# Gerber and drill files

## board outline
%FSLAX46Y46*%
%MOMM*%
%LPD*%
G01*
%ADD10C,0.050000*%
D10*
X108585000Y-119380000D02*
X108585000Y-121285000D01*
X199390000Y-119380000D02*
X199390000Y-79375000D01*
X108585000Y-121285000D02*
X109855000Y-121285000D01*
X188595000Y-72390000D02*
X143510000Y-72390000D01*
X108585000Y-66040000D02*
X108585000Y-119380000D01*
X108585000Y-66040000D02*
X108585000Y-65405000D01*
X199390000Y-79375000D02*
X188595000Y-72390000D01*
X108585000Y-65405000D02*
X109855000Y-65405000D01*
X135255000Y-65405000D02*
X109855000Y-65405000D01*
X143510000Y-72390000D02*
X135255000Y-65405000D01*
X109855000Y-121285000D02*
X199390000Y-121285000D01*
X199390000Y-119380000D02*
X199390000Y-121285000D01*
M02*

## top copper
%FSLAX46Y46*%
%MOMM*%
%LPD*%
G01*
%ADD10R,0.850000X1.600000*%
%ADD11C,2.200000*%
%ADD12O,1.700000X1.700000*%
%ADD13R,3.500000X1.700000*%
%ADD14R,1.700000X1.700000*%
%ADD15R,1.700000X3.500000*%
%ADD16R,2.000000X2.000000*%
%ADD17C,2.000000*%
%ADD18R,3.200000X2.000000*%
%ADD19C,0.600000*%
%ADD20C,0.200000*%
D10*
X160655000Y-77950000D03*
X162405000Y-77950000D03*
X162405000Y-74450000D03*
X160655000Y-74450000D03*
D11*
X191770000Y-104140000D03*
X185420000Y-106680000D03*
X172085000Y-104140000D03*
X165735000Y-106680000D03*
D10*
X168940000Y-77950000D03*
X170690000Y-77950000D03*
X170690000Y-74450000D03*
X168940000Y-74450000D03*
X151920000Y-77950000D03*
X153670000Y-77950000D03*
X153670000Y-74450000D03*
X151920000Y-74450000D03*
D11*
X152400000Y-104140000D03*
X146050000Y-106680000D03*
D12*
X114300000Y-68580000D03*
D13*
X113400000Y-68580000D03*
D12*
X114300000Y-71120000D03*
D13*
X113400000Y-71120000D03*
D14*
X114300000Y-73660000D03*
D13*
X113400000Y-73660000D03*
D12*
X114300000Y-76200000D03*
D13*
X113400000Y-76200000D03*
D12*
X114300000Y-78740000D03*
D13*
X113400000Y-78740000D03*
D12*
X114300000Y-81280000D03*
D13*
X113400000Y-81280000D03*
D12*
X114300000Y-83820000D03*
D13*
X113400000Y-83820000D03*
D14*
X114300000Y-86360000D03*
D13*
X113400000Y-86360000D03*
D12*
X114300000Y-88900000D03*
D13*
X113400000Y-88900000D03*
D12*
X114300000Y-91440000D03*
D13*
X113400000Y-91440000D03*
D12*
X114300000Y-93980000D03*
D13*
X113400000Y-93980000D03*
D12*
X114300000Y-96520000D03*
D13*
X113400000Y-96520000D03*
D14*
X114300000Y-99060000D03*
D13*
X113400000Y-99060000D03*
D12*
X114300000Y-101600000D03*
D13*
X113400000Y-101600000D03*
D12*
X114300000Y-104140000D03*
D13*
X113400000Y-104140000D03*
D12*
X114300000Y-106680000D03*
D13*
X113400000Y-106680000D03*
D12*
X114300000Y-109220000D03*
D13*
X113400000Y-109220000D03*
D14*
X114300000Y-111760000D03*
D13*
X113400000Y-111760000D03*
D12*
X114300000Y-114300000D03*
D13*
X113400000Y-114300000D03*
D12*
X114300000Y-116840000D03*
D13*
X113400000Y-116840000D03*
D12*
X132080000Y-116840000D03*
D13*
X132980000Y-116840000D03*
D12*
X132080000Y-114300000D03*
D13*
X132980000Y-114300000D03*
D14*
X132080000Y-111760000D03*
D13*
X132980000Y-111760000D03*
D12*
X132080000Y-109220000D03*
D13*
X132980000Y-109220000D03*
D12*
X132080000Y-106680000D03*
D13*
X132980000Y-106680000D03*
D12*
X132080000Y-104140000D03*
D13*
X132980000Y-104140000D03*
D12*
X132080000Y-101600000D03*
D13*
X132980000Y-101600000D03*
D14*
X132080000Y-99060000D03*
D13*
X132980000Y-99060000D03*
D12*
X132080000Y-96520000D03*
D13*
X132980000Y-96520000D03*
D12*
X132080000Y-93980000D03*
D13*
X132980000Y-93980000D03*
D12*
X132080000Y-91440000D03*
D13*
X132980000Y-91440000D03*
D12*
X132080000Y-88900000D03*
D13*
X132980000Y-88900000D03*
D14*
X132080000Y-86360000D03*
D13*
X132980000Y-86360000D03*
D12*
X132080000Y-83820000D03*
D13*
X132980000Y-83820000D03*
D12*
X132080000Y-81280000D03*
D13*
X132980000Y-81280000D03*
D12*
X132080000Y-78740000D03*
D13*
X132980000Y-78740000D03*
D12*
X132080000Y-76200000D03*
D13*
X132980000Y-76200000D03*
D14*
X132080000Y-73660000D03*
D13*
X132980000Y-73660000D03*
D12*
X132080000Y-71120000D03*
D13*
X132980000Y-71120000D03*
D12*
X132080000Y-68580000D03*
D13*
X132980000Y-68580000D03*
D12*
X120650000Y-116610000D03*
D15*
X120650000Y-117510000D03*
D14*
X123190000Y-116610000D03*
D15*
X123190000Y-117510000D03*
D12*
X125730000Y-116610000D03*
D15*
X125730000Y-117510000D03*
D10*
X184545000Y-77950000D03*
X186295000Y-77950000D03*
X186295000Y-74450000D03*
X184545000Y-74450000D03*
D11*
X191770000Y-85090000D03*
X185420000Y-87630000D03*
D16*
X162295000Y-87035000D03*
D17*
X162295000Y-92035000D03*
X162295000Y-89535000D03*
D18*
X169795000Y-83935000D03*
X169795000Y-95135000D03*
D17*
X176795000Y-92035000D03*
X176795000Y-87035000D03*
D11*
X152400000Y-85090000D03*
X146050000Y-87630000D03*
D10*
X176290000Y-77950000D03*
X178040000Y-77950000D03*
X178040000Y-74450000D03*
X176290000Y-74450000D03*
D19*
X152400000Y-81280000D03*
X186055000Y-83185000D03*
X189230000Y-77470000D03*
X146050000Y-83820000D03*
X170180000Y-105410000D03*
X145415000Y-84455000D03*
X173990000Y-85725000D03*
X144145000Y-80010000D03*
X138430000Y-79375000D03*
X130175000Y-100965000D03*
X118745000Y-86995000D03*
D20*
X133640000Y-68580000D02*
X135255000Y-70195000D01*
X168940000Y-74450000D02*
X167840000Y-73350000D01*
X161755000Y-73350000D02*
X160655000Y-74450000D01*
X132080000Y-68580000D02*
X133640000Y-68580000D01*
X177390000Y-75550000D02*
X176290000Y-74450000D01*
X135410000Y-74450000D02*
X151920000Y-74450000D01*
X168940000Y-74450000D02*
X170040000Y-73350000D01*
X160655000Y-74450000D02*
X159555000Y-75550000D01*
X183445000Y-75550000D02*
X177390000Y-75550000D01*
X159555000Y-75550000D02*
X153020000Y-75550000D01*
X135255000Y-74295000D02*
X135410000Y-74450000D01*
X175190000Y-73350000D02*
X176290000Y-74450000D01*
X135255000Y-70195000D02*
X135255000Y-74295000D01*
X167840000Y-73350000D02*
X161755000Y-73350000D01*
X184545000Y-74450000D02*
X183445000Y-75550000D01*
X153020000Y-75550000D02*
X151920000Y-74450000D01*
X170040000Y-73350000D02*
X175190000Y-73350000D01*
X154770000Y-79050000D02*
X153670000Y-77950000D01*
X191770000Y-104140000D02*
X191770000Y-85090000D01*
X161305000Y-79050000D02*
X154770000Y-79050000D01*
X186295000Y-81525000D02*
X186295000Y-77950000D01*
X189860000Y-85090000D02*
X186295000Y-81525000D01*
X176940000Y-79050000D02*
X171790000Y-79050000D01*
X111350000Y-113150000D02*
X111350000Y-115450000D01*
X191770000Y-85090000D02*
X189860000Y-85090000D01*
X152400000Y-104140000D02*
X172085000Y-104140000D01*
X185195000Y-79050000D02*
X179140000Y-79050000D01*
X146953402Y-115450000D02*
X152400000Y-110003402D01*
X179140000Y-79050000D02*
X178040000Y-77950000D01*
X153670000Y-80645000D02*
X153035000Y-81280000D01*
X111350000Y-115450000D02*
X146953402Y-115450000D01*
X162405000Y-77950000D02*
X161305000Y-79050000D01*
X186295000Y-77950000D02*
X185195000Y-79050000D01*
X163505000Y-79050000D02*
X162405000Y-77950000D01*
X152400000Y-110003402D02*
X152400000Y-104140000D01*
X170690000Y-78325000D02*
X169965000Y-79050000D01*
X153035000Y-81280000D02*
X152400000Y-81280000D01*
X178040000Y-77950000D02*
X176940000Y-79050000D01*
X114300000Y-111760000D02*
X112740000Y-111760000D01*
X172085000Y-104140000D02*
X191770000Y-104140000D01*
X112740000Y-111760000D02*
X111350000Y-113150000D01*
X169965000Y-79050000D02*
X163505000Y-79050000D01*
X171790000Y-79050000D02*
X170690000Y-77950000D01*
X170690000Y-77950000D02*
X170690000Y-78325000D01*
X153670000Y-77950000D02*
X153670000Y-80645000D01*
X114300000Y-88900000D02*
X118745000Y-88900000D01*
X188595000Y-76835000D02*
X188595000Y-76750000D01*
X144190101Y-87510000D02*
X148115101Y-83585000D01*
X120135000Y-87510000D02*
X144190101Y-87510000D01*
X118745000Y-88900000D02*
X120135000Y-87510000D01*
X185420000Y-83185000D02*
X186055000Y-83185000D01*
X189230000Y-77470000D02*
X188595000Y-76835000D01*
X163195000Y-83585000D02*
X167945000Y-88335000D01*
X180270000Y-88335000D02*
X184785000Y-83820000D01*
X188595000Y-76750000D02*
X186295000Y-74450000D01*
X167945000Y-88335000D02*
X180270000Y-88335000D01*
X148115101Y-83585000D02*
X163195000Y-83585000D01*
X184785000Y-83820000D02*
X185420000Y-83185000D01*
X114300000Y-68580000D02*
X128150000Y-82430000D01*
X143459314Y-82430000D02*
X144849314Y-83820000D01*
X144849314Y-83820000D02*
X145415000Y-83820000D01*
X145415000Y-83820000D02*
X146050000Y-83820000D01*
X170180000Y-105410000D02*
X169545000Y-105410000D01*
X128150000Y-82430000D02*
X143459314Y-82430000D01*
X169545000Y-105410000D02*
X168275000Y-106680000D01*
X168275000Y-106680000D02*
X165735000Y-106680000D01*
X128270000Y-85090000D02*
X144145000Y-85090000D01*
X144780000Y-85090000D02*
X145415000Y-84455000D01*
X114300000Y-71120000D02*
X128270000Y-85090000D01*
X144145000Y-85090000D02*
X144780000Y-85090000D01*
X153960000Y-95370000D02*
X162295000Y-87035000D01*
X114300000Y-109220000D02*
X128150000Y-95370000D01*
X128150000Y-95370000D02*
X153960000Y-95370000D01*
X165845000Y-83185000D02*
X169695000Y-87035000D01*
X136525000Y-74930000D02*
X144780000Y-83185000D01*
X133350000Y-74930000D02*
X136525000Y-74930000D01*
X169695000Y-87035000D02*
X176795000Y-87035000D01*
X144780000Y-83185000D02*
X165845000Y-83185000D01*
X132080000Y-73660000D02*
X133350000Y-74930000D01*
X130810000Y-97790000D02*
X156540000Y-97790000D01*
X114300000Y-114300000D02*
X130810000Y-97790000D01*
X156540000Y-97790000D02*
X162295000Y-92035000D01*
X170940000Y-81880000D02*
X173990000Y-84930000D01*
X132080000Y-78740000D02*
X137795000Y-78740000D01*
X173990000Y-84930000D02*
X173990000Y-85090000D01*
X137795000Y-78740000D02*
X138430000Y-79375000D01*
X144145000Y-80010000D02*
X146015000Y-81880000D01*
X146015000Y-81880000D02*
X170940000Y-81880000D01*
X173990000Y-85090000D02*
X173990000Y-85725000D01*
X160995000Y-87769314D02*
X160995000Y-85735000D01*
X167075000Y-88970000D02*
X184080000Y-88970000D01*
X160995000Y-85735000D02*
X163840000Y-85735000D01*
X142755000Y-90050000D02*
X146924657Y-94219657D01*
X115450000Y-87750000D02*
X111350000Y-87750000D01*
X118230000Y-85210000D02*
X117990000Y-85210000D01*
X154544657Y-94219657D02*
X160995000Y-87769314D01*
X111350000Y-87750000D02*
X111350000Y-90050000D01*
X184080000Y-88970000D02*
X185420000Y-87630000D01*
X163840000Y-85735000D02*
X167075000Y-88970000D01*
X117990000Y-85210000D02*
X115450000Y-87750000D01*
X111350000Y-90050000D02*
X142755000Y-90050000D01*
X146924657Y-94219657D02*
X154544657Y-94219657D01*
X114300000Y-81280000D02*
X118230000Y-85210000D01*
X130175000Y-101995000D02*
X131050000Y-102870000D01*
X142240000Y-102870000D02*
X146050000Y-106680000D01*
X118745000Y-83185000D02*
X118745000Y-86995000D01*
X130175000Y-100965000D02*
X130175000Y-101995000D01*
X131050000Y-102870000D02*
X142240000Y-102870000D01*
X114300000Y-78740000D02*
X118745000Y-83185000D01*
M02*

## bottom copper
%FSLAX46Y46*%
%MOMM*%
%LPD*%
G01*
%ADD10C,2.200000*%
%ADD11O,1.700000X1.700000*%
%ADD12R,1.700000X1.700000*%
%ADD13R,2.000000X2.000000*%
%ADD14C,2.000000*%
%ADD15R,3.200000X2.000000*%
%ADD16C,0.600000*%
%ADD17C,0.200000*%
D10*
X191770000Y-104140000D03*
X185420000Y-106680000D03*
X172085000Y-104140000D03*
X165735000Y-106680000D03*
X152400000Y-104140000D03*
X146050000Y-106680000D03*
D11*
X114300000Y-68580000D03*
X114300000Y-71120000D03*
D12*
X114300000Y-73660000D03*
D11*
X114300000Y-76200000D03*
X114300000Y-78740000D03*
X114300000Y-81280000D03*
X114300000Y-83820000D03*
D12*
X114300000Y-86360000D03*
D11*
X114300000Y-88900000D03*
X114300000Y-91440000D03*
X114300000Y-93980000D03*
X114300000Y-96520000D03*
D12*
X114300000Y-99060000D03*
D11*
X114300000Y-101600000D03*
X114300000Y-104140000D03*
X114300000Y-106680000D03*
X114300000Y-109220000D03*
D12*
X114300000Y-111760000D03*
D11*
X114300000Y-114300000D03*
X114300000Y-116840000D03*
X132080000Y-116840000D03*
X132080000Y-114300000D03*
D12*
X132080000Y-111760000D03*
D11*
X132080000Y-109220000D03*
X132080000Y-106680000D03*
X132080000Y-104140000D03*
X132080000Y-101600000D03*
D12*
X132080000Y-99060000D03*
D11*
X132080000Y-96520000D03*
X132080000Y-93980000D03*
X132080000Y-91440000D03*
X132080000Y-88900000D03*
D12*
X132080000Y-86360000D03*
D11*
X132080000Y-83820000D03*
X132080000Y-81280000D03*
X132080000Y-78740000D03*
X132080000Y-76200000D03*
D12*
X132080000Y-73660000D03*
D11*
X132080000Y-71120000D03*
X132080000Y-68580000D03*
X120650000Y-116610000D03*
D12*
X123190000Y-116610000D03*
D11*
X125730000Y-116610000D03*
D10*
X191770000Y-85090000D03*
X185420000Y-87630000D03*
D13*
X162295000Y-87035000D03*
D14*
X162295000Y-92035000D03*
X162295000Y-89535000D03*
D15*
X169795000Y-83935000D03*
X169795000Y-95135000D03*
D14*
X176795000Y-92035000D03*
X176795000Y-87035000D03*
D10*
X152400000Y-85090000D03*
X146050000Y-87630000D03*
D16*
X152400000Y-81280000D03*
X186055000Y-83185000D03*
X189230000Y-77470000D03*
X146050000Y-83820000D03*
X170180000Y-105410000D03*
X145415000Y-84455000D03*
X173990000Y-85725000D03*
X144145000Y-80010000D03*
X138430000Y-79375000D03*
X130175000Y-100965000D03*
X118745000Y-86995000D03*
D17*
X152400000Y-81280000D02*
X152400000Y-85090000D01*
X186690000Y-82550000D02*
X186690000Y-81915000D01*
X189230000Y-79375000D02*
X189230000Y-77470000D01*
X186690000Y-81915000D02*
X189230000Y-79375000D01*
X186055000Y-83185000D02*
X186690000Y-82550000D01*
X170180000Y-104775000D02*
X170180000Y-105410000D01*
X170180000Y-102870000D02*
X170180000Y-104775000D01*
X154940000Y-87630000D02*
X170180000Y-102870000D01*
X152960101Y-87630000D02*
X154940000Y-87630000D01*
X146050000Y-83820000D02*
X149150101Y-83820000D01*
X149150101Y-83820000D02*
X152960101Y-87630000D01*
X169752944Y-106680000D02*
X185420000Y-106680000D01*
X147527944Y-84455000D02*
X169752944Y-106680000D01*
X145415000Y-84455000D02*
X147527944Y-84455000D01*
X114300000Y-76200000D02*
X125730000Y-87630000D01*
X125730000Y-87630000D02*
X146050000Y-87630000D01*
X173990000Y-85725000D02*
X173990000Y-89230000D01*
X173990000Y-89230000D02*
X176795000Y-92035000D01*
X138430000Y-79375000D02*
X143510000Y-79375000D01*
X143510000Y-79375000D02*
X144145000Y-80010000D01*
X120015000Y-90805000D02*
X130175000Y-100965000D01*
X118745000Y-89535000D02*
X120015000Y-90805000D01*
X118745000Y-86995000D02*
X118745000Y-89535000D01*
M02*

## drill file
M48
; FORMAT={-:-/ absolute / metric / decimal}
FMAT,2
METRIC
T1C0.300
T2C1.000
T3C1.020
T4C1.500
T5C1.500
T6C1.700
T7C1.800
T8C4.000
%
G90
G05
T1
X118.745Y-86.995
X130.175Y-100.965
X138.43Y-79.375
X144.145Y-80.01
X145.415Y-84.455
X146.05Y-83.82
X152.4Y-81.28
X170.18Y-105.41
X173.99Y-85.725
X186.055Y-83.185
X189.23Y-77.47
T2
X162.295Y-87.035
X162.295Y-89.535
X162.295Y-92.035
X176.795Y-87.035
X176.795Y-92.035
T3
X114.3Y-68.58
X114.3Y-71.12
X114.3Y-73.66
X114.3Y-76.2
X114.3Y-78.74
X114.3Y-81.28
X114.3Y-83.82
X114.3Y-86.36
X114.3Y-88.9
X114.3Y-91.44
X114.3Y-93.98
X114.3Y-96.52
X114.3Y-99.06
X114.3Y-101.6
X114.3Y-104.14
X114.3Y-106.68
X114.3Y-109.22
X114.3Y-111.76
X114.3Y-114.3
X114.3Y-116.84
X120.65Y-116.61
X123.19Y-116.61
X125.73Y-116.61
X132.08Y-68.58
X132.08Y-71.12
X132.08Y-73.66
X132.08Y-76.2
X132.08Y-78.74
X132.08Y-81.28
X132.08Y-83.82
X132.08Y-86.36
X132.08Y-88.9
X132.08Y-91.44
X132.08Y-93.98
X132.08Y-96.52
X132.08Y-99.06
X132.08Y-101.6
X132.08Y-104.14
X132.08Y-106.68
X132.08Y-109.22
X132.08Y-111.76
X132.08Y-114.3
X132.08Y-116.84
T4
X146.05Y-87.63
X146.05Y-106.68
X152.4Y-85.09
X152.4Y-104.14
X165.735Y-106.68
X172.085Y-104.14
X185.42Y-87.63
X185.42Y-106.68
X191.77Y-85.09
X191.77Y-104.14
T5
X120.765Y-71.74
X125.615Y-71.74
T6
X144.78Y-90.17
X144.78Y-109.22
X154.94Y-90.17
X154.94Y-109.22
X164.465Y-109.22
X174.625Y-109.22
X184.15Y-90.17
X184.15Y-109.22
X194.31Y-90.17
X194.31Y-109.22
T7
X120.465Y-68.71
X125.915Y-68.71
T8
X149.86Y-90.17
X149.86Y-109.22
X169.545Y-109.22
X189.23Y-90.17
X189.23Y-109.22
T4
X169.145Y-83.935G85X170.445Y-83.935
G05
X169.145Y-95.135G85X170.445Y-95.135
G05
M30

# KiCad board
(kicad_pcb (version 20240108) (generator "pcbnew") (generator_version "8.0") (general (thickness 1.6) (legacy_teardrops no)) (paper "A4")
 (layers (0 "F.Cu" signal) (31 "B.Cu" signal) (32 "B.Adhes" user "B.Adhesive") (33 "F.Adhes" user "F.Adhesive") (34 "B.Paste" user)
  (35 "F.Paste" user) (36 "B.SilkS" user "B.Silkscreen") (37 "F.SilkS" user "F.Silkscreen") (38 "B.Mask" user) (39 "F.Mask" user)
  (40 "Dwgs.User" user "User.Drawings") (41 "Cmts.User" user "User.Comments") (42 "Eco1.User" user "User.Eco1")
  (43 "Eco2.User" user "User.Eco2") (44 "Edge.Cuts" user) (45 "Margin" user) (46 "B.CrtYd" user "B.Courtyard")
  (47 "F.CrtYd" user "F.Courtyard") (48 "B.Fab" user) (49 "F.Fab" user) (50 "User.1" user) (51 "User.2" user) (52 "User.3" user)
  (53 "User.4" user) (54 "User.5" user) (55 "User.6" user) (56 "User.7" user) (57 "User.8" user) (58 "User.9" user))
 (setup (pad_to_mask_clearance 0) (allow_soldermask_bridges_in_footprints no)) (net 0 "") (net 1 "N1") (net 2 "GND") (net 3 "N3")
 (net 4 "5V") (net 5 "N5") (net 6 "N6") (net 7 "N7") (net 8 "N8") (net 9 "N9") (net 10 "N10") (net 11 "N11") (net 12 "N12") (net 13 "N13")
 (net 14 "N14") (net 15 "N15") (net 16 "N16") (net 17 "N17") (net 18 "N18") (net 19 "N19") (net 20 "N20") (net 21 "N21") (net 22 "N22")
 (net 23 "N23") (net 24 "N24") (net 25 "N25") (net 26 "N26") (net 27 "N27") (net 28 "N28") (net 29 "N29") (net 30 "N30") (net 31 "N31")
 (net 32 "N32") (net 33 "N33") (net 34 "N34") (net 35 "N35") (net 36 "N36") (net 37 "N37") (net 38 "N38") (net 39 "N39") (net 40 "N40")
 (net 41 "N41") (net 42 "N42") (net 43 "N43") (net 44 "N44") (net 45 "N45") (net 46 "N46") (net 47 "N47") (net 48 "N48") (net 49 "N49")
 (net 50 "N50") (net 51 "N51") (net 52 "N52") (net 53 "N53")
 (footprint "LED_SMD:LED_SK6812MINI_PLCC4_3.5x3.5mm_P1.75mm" (layer "F.Cu") (at 161.53 76.2 90)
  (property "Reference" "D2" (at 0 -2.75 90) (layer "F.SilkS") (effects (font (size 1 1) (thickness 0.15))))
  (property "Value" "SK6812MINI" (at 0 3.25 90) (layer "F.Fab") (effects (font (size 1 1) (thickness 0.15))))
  (pad "1" smd rect (at -1.75 -0.875 90) (size 1.6 0.85) (layers "F.Cu" "F.Paste" "F.Mask") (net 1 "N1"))
  (pad "2" smd rect (at -1.75 0.875 90) (size 1.6 0.85) (layers "F.Cu" "F.Paste" "F.Mask") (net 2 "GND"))
  (pad "3" smd rect (at 1.75 0.875 90) (size 1.6 0.85) (layers "F.Cu" "F.Paste" "F.Mask") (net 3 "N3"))
  (pad "4" smd rect (at 1.75 -0.875 90) (size 1.6 0.85) (layers "F.Cu" "F.Paste" "F.Mask") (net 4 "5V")))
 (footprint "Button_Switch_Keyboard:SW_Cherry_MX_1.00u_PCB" (layer "F.Cu") (at 191.77 104.14)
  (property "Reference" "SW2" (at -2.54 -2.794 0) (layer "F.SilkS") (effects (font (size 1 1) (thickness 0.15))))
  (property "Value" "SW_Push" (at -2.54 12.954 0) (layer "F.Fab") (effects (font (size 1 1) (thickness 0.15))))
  (pad "" np_thru_hole circle (at -7.62 5.08) (size 1.7 1.7) (drill 1.7) (layers "*.Cu" "*.Mask"))
  (pad "" np_thru_hole circle (at -2.54 5.08) (size 4 4) (drill 4) (layers "*.Cu" "*.Mask"))
  (pad "" np_thru_hole circle (at 2.54 5.08) (size 1.7 1.7) (drill 1.7) (layers "*.Cu" "*.Mask"))
  (pad "1" thru_hole circle (at 0 0) (size 2.2 2.2) (drill 1.5) (layers "*.Cu" "*.Mask") (remove_unused_layers no) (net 2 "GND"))
  (pad "2" thru_hole circle (at -6.35 2.54) (size 2.2 2.2) (drill 1.5) (layers "*.Cu" "*.Mask") (remove_unused_layers no) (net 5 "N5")))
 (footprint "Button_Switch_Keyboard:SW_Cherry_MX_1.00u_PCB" (layer "F.Cu") (at 172.085 104.14)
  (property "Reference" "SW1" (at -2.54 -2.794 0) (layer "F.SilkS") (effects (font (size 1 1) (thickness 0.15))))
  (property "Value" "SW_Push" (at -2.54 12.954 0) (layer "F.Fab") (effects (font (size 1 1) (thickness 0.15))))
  (pad "" np_thru_hole circle (at -7.62 5.08) (size 1.7 1.7) (drill 1.7) (layers "*.Cu" "*.Mask"))
  (pad "" np_thru_hole circle (at -2.54 5.08) (size 4 4) (drill 4) (layers "*.Cu" "*.Mask"))
  (pad "" np_thru_hole circle (at 2.54 5.08) (size 1.7 1.7) (drill 1.7) (layers "*.Cu" "*.Mask"))
  (pad "1" thru_hole circle (at 0 0) (size 2.2 2.2) (drill 1.5) (layers "*.Cu" "*.Mask") (remove_unused_layers no) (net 2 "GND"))
  (pad "2" thru_hole circle (at -6.35 2.54) (size 2.2 2.2) (drill 1.5) (layers "*.Cu" "*.Mask") (remove_unused_layers no) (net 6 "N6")))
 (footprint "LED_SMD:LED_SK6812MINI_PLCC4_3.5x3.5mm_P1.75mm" (layer "F.Cu") (at 169.815 76.2 90)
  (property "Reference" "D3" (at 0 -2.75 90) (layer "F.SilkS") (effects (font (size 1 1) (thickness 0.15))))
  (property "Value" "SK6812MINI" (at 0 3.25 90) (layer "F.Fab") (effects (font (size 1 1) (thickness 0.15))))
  (pad "1" smd rect (at -1.75 -0.875 90) (size 1.6 0.85) (layers "F.Cu" "F.Paste" "F.Mask") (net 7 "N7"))
  (pad "2" smd rect (at -1.75 0.875 90) (size 1.6 0.85) (layers "F.Cu" "F.Paste" "F.Mask") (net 2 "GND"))
  (pad "3" smd rect (at 1.75 0.875 90) (size 1.6 0.85) (layers "F.Cu" "F.Paste" "F.Mask") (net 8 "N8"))
  (pad "4" smd rect (at 1.75 -0.875 90) (size 1.6 0.85) (layers "F.Cu" "F.Paste" "F.Mask") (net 4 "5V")))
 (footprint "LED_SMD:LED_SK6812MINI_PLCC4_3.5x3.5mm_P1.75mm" (layer "F.Cu") (at 152.795 76.2 90)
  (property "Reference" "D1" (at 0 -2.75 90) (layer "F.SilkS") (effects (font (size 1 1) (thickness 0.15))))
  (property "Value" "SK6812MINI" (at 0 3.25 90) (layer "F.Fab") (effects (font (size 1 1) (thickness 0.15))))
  (pad "1" smd rect (at -1.75 -0.875 90) (size 1.6 0.85) (layers "F.Cu" "F.Paste" "F.Mask") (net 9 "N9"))
  (pad "2" smd rect (at -1.75 0.875 90) (size 1.6 0.85) (layers "F.Cu" "F.Paste" "F.Mask") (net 2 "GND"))
  (pad "3" smd rect (at 1.75 0.875 90) (size 1.6 0.85) (layers "F.Cu" "F.Paste" "F.Mask") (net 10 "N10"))
  (pad "4" smd rect (at 1.75 -0.875 90) (size 1.6 0.85) (layers "F.Cu" "F.Paste" "F.Mask") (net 4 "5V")))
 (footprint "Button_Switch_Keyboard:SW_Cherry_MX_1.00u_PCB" (layer "F.Cu") (at 152.4 104.14)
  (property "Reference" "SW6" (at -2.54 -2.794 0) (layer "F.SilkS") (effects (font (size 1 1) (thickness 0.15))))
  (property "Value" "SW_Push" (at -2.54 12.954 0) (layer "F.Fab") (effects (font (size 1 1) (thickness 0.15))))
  (pad "" np_thru_hole circle (at -7.62 5.08) (size 1.7 1.7) (drill 1.7) (layers "*.Cu" "*.Mask"))
  (pad "" np_thru_hole circle (at -2.54 5.08) (size 4 4) (drill 4) (layers "*.Cu" "*.Mask"))
  (pad "" np_thru_hole circle (at 2.54 5.08) (size 1.7 1.7) (drill 1.7) (layers "*.Cu" "*.Mask"))
  (pad "1" thru_hole circle (at 0 0) (size 2.2 2.2) (drill 1.5) (layers "*.Cu" "*.Mask") (remove_unused_layers no) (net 2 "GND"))
  (pad "2" thru_hole circle (at -6.35 2.54) (size 2.2 2.2) (drill 1.5) (layers "*.Cu" "*.Mask") (remove_unused_layers no) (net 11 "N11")))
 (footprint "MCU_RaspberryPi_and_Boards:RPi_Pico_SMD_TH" (layer "F.Cu") (at 123.19 92.71)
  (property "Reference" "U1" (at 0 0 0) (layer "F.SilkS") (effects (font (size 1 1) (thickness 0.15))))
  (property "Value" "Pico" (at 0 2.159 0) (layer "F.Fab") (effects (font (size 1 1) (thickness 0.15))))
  (pad "" np_thru_hole oval (at -2.725 -24) (size 1.8 1.8) (drill 1.8) (layers "*.Cu" "*.Mask"))
  (pad "" np_thru_hole oval (at -2.425 -20.97) (size 1.5 1.5) (drill 1.5) (layers "*.Cu" "*.Mask"))
  (pad "" np_thru_hole oval (at 2.425 -20.97) (size 1.5 1.5) (drill 1.5) (layers "*.Cu" "*.Mask"))
  (pad "" np_thru_hole oval (at 2.725 -24) (size 1.8 1.8) (drill 1.8) (layers "*.Cu" "*.Mask"))
  (pad "1" thru_hole oval (at -8.89 -24.13) (size 1.7 1.7) (drill 1.02) (layers "*.Cu" "*.Mask") (remove_unused_layers no) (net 6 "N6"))
  (pad "1" smd rect (at -8.89 -24.13) (size 3.5 1.7) (drill (offset -0.9 0)) (layers "F.Cu" "F.Mask") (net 6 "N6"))
  (pad "2" thru_hole oval (at -8.89 -21.59) (size 1.7 1.7) (drill 1.02) (layers "*.Cu" "*.Mask") (remove_unused_layers no) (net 5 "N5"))
  (pad "2" smd rect (at -8.89 -21.59) (size 3.5 1.7) (drill (offset -0.9 0)) (layers "F.Cu" "F.Mask") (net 5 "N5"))
  (pad "3" thru_hole rect (at -8.89 -19.05) (size 1.7 1.7) (drill 1.02) (layers "*.Cu" "*.Mask") (remove_unused_layers no) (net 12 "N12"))
  (pad "3" smd rect (at -8.89 -19.05) (size 3.5 1.7) (drill (offset -0.9 0)) (layers "F.Cu" "F.Mask") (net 12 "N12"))
  (pad "4" thru_hole oval (at -8.89 -16.51) (size 1.7 1.7) (drill 1.02) (layers "*.Cu" "*.Mask") (remove_unused_layers no) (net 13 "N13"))
  (pad "4" smd rect (at -8.89 -16.51) (size 3.5 1.7) (drill (offset -0.9 0)) (layers "F.Cu" "F.Mask") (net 13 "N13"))
  (pad "5" thru_hole oval (at -8.89 -13.97) (size 1.7 1.7) (drill 1.02) (layers "*.Cu" "*.Mask") (remove_unused_layers no) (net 11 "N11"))
  (pad "5" smd rect (at -8.89 -13.97) (size 3.5 1.7) (drill (offset -0.9 0)) (layers "F.Cu" "F.Mask") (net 11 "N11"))
  (pad "6" thru_hole oval (at -8.89 -11.43) (size 1.7 1.7) (drill 1.02) (layers "*.Cu" "*.Mask") (remove_unused_layers no) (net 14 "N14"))
  (pad "6" smd rect (at -8.89 -11.43) (size 3.5 1.7) (drill (offset -0.9 0)) (layers "F.Cu" "F.Mask") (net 14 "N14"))
  (pad "7" thru_hole oval (at -8.89 -8.89) (size 1.7 1.7) (drill 1.02) (layers "*.Cu" "*.Mask") (remove_unused_layers no) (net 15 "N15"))
  (pad "7" smd rect (at -8.89 -8.89) (size 3.5 1.7) (drill (offset -0.9 0)) (layers "F.Cu" "F.Mask") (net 15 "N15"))
  (pad "8" thru_hole rect (at -8.89 -6.35) (size 1.7 1.7) (drill 1.02) (layers "*.Cu" "*.Mask") (remove_unused_layers no) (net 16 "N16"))
  (pad "8" smd rect (at -8.89 -6.35) (size 3.5 1.7) (drill (offset -0.9 0)) (layers "F.Cu" "F.Mask") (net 16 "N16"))
  (pad "9" thru_hole oval (at -8.89 -3.81) (size 1.7 1.7) (drill 1.02) (layers "*.Cu" "*.Mask") (remove_unused_layers no) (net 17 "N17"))
  (pad "9" smd rect (at -8.89 -3.81) (size 3.5 1.7) (drill (offset -0.9 0)) (layers "F.Cu" "F.Mask") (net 17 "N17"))
  (pad "10" thru_hole oval (at -8.89 -1.27) (size 1.7 1.7) (drill 1.02) (layers "*.Cu" "*.Mask") (remove_unused_layers no) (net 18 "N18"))
  (pad "10" smd rect (at -8.89 -1.27) (size 3.5 1.7) (drill (offset -0.9 0)) (layers "F.Cu" "F.Mask") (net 18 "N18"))
  (pad "11" thru_hole oval (at -8.89 1.27) (size 1.7 1.7) (drill 1.02) (layers "*.Cu" "*.Mask") (remove_unused_layers no) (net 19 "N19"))
  (pad "11" smd rect (at -8.89 1.27) (size 3.5 1.7) (drill (offset -0.9 0)) (layers "F.Cu" "F.Mask") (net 19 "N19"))
  (pad "12" thru_hole oval (at -8.89 3.81) (size 1.7 1.7) (drill 1.02) (layers "*.Cu" "*.Mask") (remove_unused_layers no) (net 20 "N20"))
  (pad "12" smd rect (at -8.89 3.81) (size 3.5 1.7) (drill (offset -0.9 0)) (layers "F.Cu" "F.Mask") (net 20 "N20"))
  (pad "13" thru_hole rect (at -8.89 6.35) (size 1.7 1.7) (drill 1.02) (layers "*.Cu" "*.Mask") (remove_unused_layers no) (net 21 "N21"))
  (pad "13" smd rect (at -8.89 6.35) (size 3.5 1.7) (drill (offset -0.9 0)) (layers "F.Cu" "F.Mask") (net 21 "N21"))
  (pad "14" thru_hole oval (at -8.89 8.89) (size 1.7 1.7) (drill 1.02) (layers "*.Cu" "*.Mask") (remove_unused_layers no) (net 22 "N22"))
  (pad "14" smd rect (at -8.89 8.89) (size 3.5 1.7) (drill (offset -0.9 0)) (layers "F.Cu" "F.Mask") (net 22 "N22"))
  (pad "15" thru_hole oval (at -8.89 11.43) (size 1.7 1.7) (drill 1.02) (layers "*.Cu" "*.Mask") (remove_unused_layers no) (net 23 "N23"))
  (pad "15" smd rect (at -8.89 11.43) (size 3.5 1.7) (drill (offset -0.9 0)) (layers "F.Cu" "F.Mask") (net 23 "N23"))
  (pad "16" thru_hole oval (at -8.89 13.97) (size 1.7 1.7) (drill 1.02) (layers "*.Cu" "*.Mask") (remove_unused_layers no) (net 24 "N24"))
  (pad "16" smd rect (at -8.89 13.97) (size 3.5 1.7) (drill (offset -0.9 0)) (layers "F.Cu" "F.Mask") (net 24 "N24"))
  (pad "17" thru_hole oval (at -8.89 16.51) (size 1.7 1.7) (drill 1.02) (layers "*.Cu" "*.Mask") (remove_unused_layers no) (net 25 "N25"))
  (pad "17" smd rect (at -8.89 16.51) (size 3.5 1.7) (drill (offset -0.9 0)) (layers "F.Cu" "F.Mask") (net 25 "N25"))
  (pad "18" thru_hole rect (at -8.89 19.05) (size 1.7 1.7) (drill 1.02) (layers "*.Cu" "*.Mask") (remove_unused_layers no) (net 2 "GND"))
  (pad "18" smd rect (at -8.89 19.05) (size 3.5 1.7) (drill (offset -0.9 0)) (layers "F.Cu" "F.Mask") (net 2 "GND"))
  (pad "19" thru_hole oval (at -8.89 21.59) (size 1.7 1.7) (drill 1.02) (layers "*.Cu" "*.Mask") (remove_unused_layers no) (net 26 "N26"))
  (pad "19" smd rect (at -8.89 21.59) (size 3.5 1.7) (drill (offset -0.9 0)) (layers "F.Cu" "F.Mask") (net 26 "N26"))
  (pad "20" thru_hole oval (at -8.89 24.13) (size 1.7 1.7) (drill 1.02) (layers "*.Cu" "*.Mask") (remove_unused_layers no) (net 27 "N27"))
  (pad "20" smd rect (at -8.89 24.13) (size 3.5 1.7) (drill (offset -0.9 0)) (layers "F.Cu" "F.Mask") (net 27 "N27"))
  (pad "21" thru_hole oval (at 8.89 24.13) (size 1.7 1.7) (drill 1.02) (layers "*.Cu" "*.Mask") (remove_unused_layers no) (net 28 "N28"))
  (pad "21" smd rect (at 8.89 24.13) (size 3.5 1.7) (drill (offset 0.9 0)) (layers "F.Cu" "F.Mask") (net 28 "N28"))
  (pad "22" thru_hole oval (at 8.89 21.59) (size 1.7 1.7) (drill 1.02) (layers "*.Cu" "*.Mask") (remove_unused_layers no) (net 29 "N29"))
  (pad "22" smd rect (at 8.89 21.59) (size 3.5 1.7) (drill (offset 0.9 0)) (layers "F.Cu" "F.Mask") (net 29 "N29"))
  (pad "23" thru_hole rect (at 8.89 19.05) (size 1.7 1.7) (drill 1.02) (layers "*.Cu" "*.Mask") (remove_unused_layers no) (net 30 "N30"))
  (pad "23" smd rect (at 8.89 19.05) (size 3.5 1.7) (drill (offset 0.9 0)) (layers "F.Cu" "F.Mask") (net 30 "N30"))
  (pad "24" thru_hole oval (at 8.89 16.51) (size 1.7 1.7) (drill 1.02) (layers "*.Cu" "*.Mask") (remove_unused_layers no) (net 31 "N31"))
  (pad "24" smd rect (at 8.89 16.51) (size 3.5 1.7) (drill (offset 0.9 0)) (layers "F.Cu" "F.Mask") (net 31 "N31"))
  (pad "25" thru_hole oval (at 8.89 13.97) (size 1.7 1.7) (drill 1.02) (layers "*.Cu" "*.Mask") (remove_unused_layers no) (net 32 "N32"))
  (pad "25" smd rect (at 8.89 13.97) (size 3.5 1.7) (drill (offset 0.9 0)) (layers "F.Cu" "F.Mask") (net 32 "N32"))
  (pad "26" thru_hole oval (at 8.89 11.43) (size 1.7 1.7) (drill 1.02) (layers "*.Cu" "*.Mask") (remove_unused_layers no) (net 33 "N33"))
  (pad "26" smd rect (at 8.89 11.43) (size 3.5 1.7) (drill (offset 0.9 0)) (layers "F.Cu" "F.Mask") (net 33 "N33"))
  (pad "27" thru_hole oval (at 8.89 8.89) (size 1.7 1.7) (drill 1.02) (layers "*.Cu" "*.Mask") (remove_unused_layers no) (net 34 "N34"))
  (pad "27" smd rect (at 8.89 8.89) (size 3.5 1.7) (drill (offset 0.9 0)) (layers "F.Cu" "F.Mask") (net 34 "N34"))
  (pad "28" thru_hole rect (at 8.89 6.35) (size 1.7 1.7) (drill 1.02) (layers "*.Cu" "*.Mask") (remove_unused_layers no) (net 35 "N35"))
  (pad "28" smd rect (at 8.89 6.35) (size 3.5 1.7) (drill (offset 0.9 0)) (layers "F.Cu" "F.Mask") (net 35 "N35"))
  (pad "29" thru_hole oval (at 8.89 3.81) (size 1.7 1.7) (drill 1.02) (layers "*.Cu" "*.Mask") (remove_unused_layers no) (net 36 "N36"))
  (pad "29" smd rect (at 8.89 3.81) (size 3.5 1.7) (drill (offset 0.9 0)) (layers "F.Cu" "F.Mask") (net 36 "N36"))
  (pad "30" thru_hole oval (at 8.89 1.27) (size 1.7 1.7) (drill 1.02) (layers "*.Cu" "*.Mask") (remove_unused_layers no) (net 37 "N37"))
  (pad "30" smd rect (at 8.89 1.27) (size 3.5 1.7) (drill (offset 0.9 0)) (layers "F.Cu" "F.Mask") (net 37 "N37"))
  (pad "31" thru_hole oval (at 8.89 -1.27) (size 1.7 1.7) (drill 1.02) (layers "*.Cu" "*.Mask") (remove_unused_layers no) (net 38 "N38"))
  (pad "31" smd rect (at 8.89 -1.27) (size 3.5 1.7) (drill (offset 0.9 0)) (layers "F.Cu" "F.Mask") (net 38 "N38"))
  (pad "32" thru_hole oval (at 8.89 -3.81) (size 1.7 1.7) (drill 1.02) (layers "*.Cu" "*.Mask") (remove_unused_layers no) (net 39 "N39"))
  (pad "32" smd rect (at 8.89 -3.81) (size 3.5 1.7) (drill (offset 0.9 0)) (layers "F.Cu" "F.Mask") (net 39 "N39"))
  (pad "33" thru_hole rect (at 8.89 -6.35) (size 1.7 1.7) (drill 1.02) (layers "*.Cu" "*.Mask") (remove_unused_layers no) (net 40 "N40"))
  (pad "33" smd rect (at 8.89 -6.35) (size 3.5 1.7) (drill (offset 0.9 0)) (layers "F.Cu" "F.Mask") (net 40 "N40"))
  (pad "34" thru_hole oval (at 8.89 -8.89) (size 1.7 1.7) (drill 1.02) (layers "*.Cu" "*.Mask") (remove_unused_layers no) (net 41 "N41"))
  (pad "34" smd rect (at 8.89 -8.89) (size 3.5 1.7) (drill (offset 0.9 0)) (layers "F.Cu" "F.Mask") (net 41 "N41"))
  (pad "35" thru_hole oval (at 8.89 -11.43) (size 1.7 1.7) (drill 1.02) (layers "*.Cu" "*.Mask") (remove_unused_layers no) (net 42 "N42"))
  (pad "35" smd rect (at 8.89 -11.43) (size 3.5 1.7) (drill (offset 0.9 0)) (layers "F.Cu" "F.Mask") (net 42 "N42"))
  (pad "36" thru_hole oval (at 8.89 -13.97) (size 1.7 1.7) (drill 1.02) (layers "*.Cu" "*.Mask") (remove_unused_layers no) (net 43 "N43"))
  (pad "36" smd rect (at 8.89 -13.97) (size 3.5 1.7) (drill (offset 0.9 0)) (layers "F.Cu" "F.Mask") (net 43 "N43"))
  (pad "37" thru_hole oval (at 8.89 -16.51) (size 1.7 1.7) (drill 1.02) (layers "*.Cu" "*.Mask") (remove_unused_layers no) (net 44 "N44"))
  (pad "37" smd rect (at 8.89 -16.51) (size 3.5 1.7) (drill (offset 0.9 0)) (layers "F.Cu" "F.Mask") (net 44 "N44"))
  (pad "38" thru_hole rect (at 8.89 -19.05) (size 1.7 1.7) (drill 1.02) (layers "*.Cu" "*.Mask") (remove_unused_layers no) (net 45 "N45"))
  (pad "38" smd rect (at 8.89 -19.05) (size 3.5 1.7) (drill (offset 0.9 0)) (layers "F.Cu" "F.Mask") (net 45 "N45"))
  (pad "39" thru_hole oval (at 8.89 -21.59) (size 1.7 1.7) (drill 1.02) (layers "*.Cu" "*.Mask") (remove_unused_layers no) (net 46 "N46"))
  (pad "39" smd rect (at 8.89 -21.59) (size 3.5 1.7) (drill (offset 0.9 0)) (layers "F.Cu" "F.Mask") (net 46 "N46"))
  (pad "40" thru_hole oval (at 8.89 -24.13) (size 1.7 1.7) (drill 1.02) (layers "*.Cu" "*.Mask") (remove_unused_layers no) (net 4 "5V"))
  (pad "40" smd rect (at 8.89 -24.13) (size 3.5 1.7) (drill (offset 0.9 0)) (layers "F.Cu" "F.Mask") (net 4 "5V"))
  (pad "41" thru_hole oval (at -2.54 23.9) (size 1.7 1.7) (drill 1.02) (layers "*.Cu" "*.Mask") (remove_unused_layers no) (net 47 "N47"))
  (pad "41" smd rect (at -2.54 23.9 90) (size 3.5 1.7) (drill (offset -0.9 0)) (layers "F.Cu" "F.Mask") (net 47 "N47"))
  (pad "42" thru_hole rect (at 0 23.9) (size 1.7 1.7) (drill 1.02) (layers "*.Cu" "*.Mask") (remove_unused_layers no) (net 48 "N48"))
  (pad "42" smd rect (at 0 23.9 90) (size 3.5 1.7) (drill (offset -0.9 0)) (layers "F.Cu" "F.Mask") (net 48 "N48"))
  (pad "43" thru_hole oval (at 2.54 23.9) (size 1.7 1.7) (drill 1.02) (layers "*.Cu" "*.Mask") (remove_unused_layers no) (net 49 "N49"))
  (pad "43" smd rect (at 2.54 23.9 90) (size 3.5 1.7) (drill (offset -0.9 0)) (layers "F.Cu" "F.Mask") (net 49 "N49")))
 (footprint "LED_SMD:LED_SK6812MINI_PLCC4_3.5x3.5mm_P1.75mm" (layer "F.Cu") (at 185.42 76.2 90)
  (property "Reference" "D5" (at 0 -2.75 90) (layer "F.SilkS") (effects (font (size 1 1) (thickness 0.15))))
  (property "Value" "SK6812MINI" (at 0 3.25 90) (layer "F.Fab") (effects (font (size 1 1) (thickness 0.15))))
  (pad "1" smd rect (at -1.75 -0.875 90) (size 1.6 0.85) (layers "F.Cu" "F.Paste" "F.Mask") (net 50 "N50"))
  (pad "2" smd rect (at -1.75 0.875 90) (size 1.6 0.85) (layers "F.Cu" "F.Paste" "F.Mask") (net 2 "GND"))
  (pad "3" smd rect (at 1.75 0.875 90) (size 1.6 0.85) (layers "F.Cu" "F.Paste" "F.Mask") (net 17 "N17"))
  (pad "4" smd rect (at 1.75 -0.875 90) (size 1.6 0.85) (layers "F.Cu" "F.Paste" "F.Mask") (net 4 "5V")))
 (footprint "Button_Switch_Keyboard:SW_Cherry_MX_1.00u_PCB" (layer "F.Cu") (at 191.77 85.09)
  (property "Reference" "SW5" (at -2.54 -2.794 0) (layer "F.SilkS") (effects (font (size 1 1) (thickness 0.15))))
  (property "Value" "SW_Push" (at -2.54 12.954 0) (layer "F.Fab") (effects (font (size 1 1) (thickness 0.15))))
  (pad "" np_thru_hole circle (at -7.62 5.08) (size 1.7 1.7) (drill 1.7) (layers "*.Cu" "*.Mask"))
  (pad "" np_thru_hole circle (at -2.54 5.08) (size 4 4) (drill 4) (layers "*.Cu" "*.Mask"))
  (pad "" np_thru_hole circle (at 2.54 5.08) (size 1.7 1.7) (drill 1.7) (layers "*.Cu" "*.Mask"))
  (pad "1" thru_hole circle (at 0 0) (size 2.2 2.2) (drill 1.5) (layers "*.Cu" "*.Mask") (remove_unused_layers no) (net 2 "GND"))
  (pad "2" thru_hole circle (at -6.35 2.54) (size 2.2 2.2) (drill 1.5) (layers "*.Cu" "*.Mask") (remove_unused_layers no) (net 14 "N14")))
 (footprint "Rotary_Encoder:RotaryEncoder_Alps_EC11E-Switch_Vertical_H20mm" (layer "F.Cu") (at 162.295 87.035)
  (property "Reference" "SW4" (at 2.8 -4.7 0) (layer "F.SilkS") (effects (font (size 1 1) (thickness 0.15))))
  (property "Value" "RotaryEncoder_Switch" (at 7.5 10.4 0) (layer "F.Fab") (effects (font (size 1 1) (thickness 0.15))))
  (pad "A" thru_hole rect (at 0 0) (size 2 2) (drill 1) (layers "*.Cu" "*.Mask") (remove_unused_layers no) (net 25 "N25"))
  (pad "B" thru_hole circle (at 0 5) (size 2 2) (drill 1) (layers "*.Cu" "*.Mask") (remove_unused_layers no) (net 26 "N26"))
  (pad "C" thru_hole circle (at 0 2.5) (size 2 2) (drill 1) (layers "*.Cu" "*.Mask") (remove_unused_layers no) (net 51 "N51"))
  (pad "MP" thru_hole rect (at 7.5 -3.1) (size 3.2 2) (drill oval 2.8 1.5) (layers "*.Cu" "*.Mask") (remove_unused_layers no))
  (pad "MP" thru_hole rect (at 7.5 8.1) (size 3.2 2) (drill oval 2.8 1.5) (layers "*.Cu" "*.Mask") (remove_unused_layers no))
  (pad "S1" thru_hole circle (at 14.5 5) (size 2 2) (drill 1) (layers "*.Cu" "*.Mask") (remove_unused_layers no) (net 43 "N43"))
  (pad "S2" thru_hole circle (at 14.5 0) (size 2 2) (drill 1) (layers "*.Cu" "*.Mask") (remove_unused_layers no) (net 45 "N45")))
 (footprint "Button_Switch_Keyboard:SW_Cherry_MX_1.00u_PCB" (layer "F.Cu") (at 152.4 85.09)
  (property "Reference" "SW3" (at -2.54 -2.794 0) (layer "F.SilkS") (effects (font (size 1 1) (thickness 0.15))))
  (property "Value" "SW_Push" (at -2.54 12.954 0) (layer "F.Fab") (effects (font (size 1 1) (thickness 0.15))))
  (pad "" np_thru_hole circle (at -7.62 5.08) (size 1.7 1.7) (drill 1.7) (layers "*.Cu" "*.Mask"))
  (pad "" np_thru_hole circle (at -2.54 5.08) (size 4 4) (drill 4) (layers "*.Cu" "*.Mask"))
  (pad "" np_thru_hole circle (at 2.54 5.08) (size 1.7 1.7) (drill 1.7) (layers "*.Cu" "*.Mask"))
  (pad "1" thru_hole circle (at 0 0) (size 2.2 2.2) (drill 1.5) (layers "*.Cu" "*.Mask") (remove_unused_layers no) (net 2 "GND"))
  (pad "2" thru_hole circle (at -6.35 2.54) (size 2.2 2.2) (drill 1.5) (layers "*.Cu" "*.Mask") (remove_unused_layers no) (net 13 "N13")))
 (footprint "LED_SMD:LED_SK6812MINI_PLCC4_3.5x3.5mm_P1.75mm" (layer "F.Cu") (at 177.165 76.2 90)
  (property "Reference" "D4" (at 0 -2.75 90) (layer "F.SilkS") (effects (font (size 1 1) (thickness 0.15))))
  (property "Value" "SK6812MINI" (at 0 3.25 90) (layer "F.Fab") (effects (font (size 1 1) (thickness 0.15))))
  (pad "1" smd rect (at -1.75 -0.875 90) (size 1.6 0.85) (layers "F.Cu" "F.Paste" "F.Mask") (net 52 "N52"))
  (pad "2" smd rect (at -1.75 0.875 90) (size 1.6 0.85) (layers "F.Cu" "F.Paste" "F.Mask") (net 2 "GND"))
  (pad "3" smd rect (at 1.75 0.875 90) (size 1.6 0.85) (layers "F.Cu" "F.Paste" "F.Mask") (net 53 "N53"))
  (pad "4" smd rect (at 1.75 -0.875 90) (size 1.6 0.85) (layers "F.Cu" "F.Paste" "F.Mask") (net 4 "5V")))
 (gr_line (start 108.585 119.38) (end 108.585 121.285) (stroke (width 0.05) (type default)) (layer "Edge.Cuts"))
 (gr_line (start 199.39 119.38) (end 199.39 79.375) (stroke (width 0.05) (type default)) (layer "Edge.Cuts"))
 (gr_line (start 108.585 121.285) (end 109.855 121.285) (stroke (width 0.05) (type default)) (layer "Edge.Cuts"))
 (gr_line (start 188.595 72.39) (end 143.51 72.39) (stroke (width 0.05) (type default)) (layer "Edge.Cuts"))
 (gr_line (start 108.585 66.04) (end 108.585 119.38) (stroke (width 0.05) (type default)) (layer "Edge.Cuts"))
 (gr_line (start 108.585 66.04) (end 108.585 65.405) (stroke (width 0.05) (type default)) (layer "Edge.Cuts"))
 (gr_line (start 199.39 79.375) (end 188.595 72.39) (stroke (width 0.05) (type default)) (layer "Edge.Cuts"))
 (gr_line (start 108.585 65.405) (end 109.855 65.405) (stroke (width 0.05) (type default)) (layer "Edge.Cuts"))
 (gr_line (start 135.255 65.405) (end 109.855 65.405) (stroke (width 0.05) (type default)) (layer "Edge.Cuts"))
 (gr_line (start 143.51 72.39) (end 135.255 65.405) (stroke (width 0.05) (type default)) (layer "Edge.Cuts"))
 (gr_line (start 109.855 121.285) (end 199.39 121.285) (stroke (width 0.05) (type default)) (layer "Edge.Cuts"))
 (gr_line (start 199.39 119.38) (end 199.39 121.285) (stroke (width 0.05) (type default)) (layer "Edge.Cuts"))
 (segment (start 133.64 68.58) (end 135.255 70.195) (width 0.2) (layer "F.Cu") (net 4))
 (segment (start 168.94 74.45) (end 167.84 73.35) (width 0.2) (layer "F.Cu") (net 4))
 (segment (start 161.755 73.35) (end 160.655 74.45) (width 0.2) (layer "F.Cu") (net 4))
 (segment (start 132.08 68.58) (end 133.64 68.58) (width 0.2) (layer "F.Cu") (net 4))
 (segment (start 177.39 75.55) (end 176.29 74.45) (width 0.2) (layer "F.Cu") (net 4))
 (segment (start 135.41 74.45) (end 151.92 74.45) (width 0.2) (layer "F.Cu") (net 4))
 (segment (start 168.94 74.45) (end 170.04 73.35) (width 0.2) (layer "F.Cu") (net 4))
 (segment (start 160.655 74.45) (end 159.555 75.55) (width 0.2) (layer "F.Cu") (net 4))
 (segment (start 183.445 75.55) (end 177.39 75.55) (width 0.2) (layer "F.Cu") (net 4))
 (segment (start 159.555 75.55) (end 153.02 75.55) (width 0.2) (layer "F.Cu") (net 4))
 (segment (start 135.255 74.295) (end 135.41 74.45) (width 0.2) (layer "F.Cu") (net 4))
 (segment (start 175.19 73.35) (end 176.29 74.45) (width 0.2) (layer "F.Cu") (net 4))
 (segment (start 135.255 70.195) (end 135.255 74.295) (width 0.2) (layer "F.Cu") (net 4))
 (segment (start 167.84 73.35) (end 161.755 73.35) (width 0.2) (layer "F.Cu") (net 4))
 (segment (start 184.545 74.45) (end 183.445 75.55) (width 0.2) (layer "F.Cu") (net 4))
 (segment (start 153.02 75.55) (end 151.92 74.45) (width 0.2) (layer "F.Cu") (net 4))
 (segment (start 170.04 73.35) (end 175.19 73.35) (width 0.2) (layer "F.Cu") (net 4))
 (segment (start 154.77 79.05) (end 153.67 77.95) (width 0.2) (layer "F.Cu") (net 2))
 (segment (start 191.77 104.14) (end 191.77 85.09) (width 0.2) (layer "F.Cu") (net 2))
 (segment (start 161.305 79.05) (end 154.77 79.05) (width 0.2) (layer "F.Cu") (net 2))
 (segment (start 186.295 81.525) (end 186.295 77.95) (width 0.2) (layer "F.Cu") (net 2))
 (segment (start 189.86 85.09) (end 186.295 81.525) (width 0.2) (layer "F.Cu") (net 2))
 (segment (start 176.94 79.05) (end 171.79 79.05) (width 0.2) (layer "F.Cu") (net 2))
 (segment (start 111.35 113.15) (end 111.35 115.45) (width 0.2) (layer "F.Cu") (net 2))
 (segment (start 191.77 85.09) (end 189.86 85.09) (width 0.2) (layer "F.Cu") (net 2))
 (segment (start 152.4 104.14) (end 172.085 104.14) (width 0.2) (layer "F.Cu") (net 2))
 (segment (start 185.195 79.05) (end 179.14 79.05) (width 0.2) (layer "F.Cu") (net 2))
 (segment (start 146.953402 115.45) (end 152.4 110.003402) (width 0.2) (layer "F.Cu") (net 2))
 (segment (start 179.14 79.05) (end 178.04 77.95) (width 0.2) (layer "F.Cu") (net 2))
 (segment (start 153.67 80.645) (end 153.035 81.28) (width 0.2) (layer "F.Cu") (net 2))
 (segment (start 111.35 115.45) (end 146.953402 115.45) (width 0.2) (layer "F.Cu") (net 2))
 (segment (start 162.405 77.95) (end 161.305 79.05) (width 0.2) (layer "F.Cu") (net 2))
 (segment (start 186.295 77.95) (end 185.195 79.05) (width 0.2) (layer "F.Cu") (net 2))
 (segment (start 163.505 79.05) (end 162.405 77.95) (width 0.2) (layer "F.Cu") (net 2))
 (segment (start 152.4 110.003402) (end 152.4 104.14) (width 0.2) (layer "F.Cu") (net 2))
 (segment (start 170.69 78.325) (end 169.965 79.05) (width 0.2) (layer "F.Cu") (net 2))
 (segment (start 153.035 81.28) (end 152.4 81.28) (width 0.2) (layer "F.Cu") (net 2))
 (segment (start 178.04 77.95) (end 176.94 79.05) (width 0.2) (layer "F.Cu") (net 2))
 (segment (start 114.3 111.76) (end 112.74 111.76) (width 0.2) (layer "F.Cu") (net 2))
 (segment (start 172.085 104.14) (end 191.77 104.14) (width 0.2) (layer "F.Cu") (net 2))
 (segment (start 112.74 111.76) (end 111.35 113.15) (width 0.2) (layer "F.Cu") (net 2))
 (segment (start 169.965 79.05) (end 163.505 79.05) (width 0.2) (layer "F.Cu") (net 2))
 (segment (start 171.79 79.05) (end 170.69 77.95) (width 0.2) (layer "F.Cu") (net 2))
 (segment (start 170.69 77.95) (end 170.69 78.325) (width 0.2) (layer "F.Cu") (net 2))
 (segment (start 153.67 77.95) (end 153.67 80.645) (width 0.2) (layer "F.Cu") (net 2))
 (via (at 152.4 81.28) (size 0.6) (drill 0.3) (layers "F.Cu" "B.Cu") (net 2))
 (segment (start 152.4 81.28) (end 152.4 85.09) (width 0.2) (layer "B.Cu") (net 2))
 (segment (start 114.3 88.9) (end 118.745 88.9) (width 0.2) (layer "F.Cu") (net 17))
 (segment (start 188.595 76.835) (end 188.595 76.75) (width 0.2) (layer "F.Cu") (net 17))
 (segment (start 144.190101 87.51) (end 148.115101 83.585) (width 0.2) (layer "F.Cu") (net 17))
 (segment (start 120.135 87.51) (end 144.190101 87.51) (width 0.2) (layer "F.Cu") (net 17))
 (segment (start 118.745 88.9) (end 120.135 87.51) (width 0.2) (layer "F.Cu") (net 17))
 (segment (start 185.42 83.185) (end 186.055 83.185) (width 0.2) (layer "F.Cu") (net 17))
 (segment (start 189.23 77.47) (end 188.595 76.835) (width 0.2) (layer "F.Cu") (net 17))
 (segment (start 163.195 83.585) (end 167.945 88.335) (width 0.2) (layer "F.Cu") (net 17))
 (segment (start 180.27 88.335) (end 184.785 83.82) (width 0.2) (layer "F.Cu") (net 17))
 (segment (start 188.595 76.75) (end 186.295 74.45) (width 0.2) (layer "F.Cu") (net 17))
 (segment (start 167.945 88.335) (end 180.27 88.335) (width 0.2) (layer "F.Cu") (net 17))
 (segment (start 148.115101 83.585) (end 163.195 83.585) (width 0.2) (layer "F.Cu") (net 17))
 (segment (start 184.785 83.82) (end 185.42 83.185) (width 0.2) (layer "F.Cu") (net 17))
 (via (at 186.055 83.185) (size 0.6) (drill 0.3) (layers "F.Cu" "B.Cu") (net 17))
 (via (at 189.23 77.47) (size 0.6) (drill 0.3) (layers "F.Cu" "B.Cu") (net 17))
 (segment (start 186.69 82.55) (end 186.69 81.915) (width 0.2) (layer "B.Cu") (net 17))
 (segment (start 189.23 79.375) (end 189.23 77.47) (width 0.2) (layer "B.Cu") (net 17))
 (segment (start 186.69 81.915) (end 189.23 79.375) (width 0.2) (layer "B.Cu") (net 17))
 (segment (start 186.055 83.185) (end 186.69 82.55) (width 0.2) (layer "B.Cu") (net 17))
 (segment (start 114.3 68.58) (end 128.15 82.43) (width 0.2) (layer "F.Cu") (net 6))
 (segment (start 143.459314 82.43) (end 144.849314 83.82) (width 0.2) (layer "F.Cu") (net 6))
 (segment (start 144.849314 83.82) (end 145.415 83.82) (width 0.2) (layer "F.Cu") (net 6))
 (segment (start 145.415 83.82) (end 146.05 83.82) (width 0.2) (layer "F.Cu") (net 6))
 (segment (start 170.18 105.41) (end 169.545 105.41) (width 0.2) (layer "F.Cu") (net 6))
 (segment (start 128.15 82.43) (end 143.459314 82.43) (width 0.2) (layer "F.Cu") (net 6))
 (segment (start 169.545 105.41) (end 168.275 106.68) (width 0.2) (layer "F.Cu") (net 6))
 (segment (start 168.275 106.68) (end 165.735 106.68) (width 0.2) (layer "F.Cu") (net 6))
 (via (at 146.05 83.82) (size 0.6) (drill 0.3) (layers "F.Cu" "B.Cu") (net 6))
 (via (at 170.18 105.41) (size 0.6) (drill 0.3) (layers "F.Cu" "B.Cu") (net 6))
 (segment (start 170.18 104.775) (end 170.18 105.41) (width 0.2) (layer "B.Cu") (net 6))
 (segment (start 170.18 102.87) (end 170.18 104.775) (width 0.2) (layer "B.Cu") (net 6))
 (segment (start 154.94 87.63) (end 170.18 102.87) (width 0.2) (layer "B.Cu") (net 6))
 (segment (start 152.960101 87.63) (end 154.94 87.63) (width 0.2) (layer "B.Cu") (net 6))
 (segment (start 146.05 83.82) (end 149.150101 83.82) (width 0.2) (layer "B.Cu") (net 6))
 (segment (start 149.150101 83.82) (end 152.960101 87.63) (width 0.2) (layer "B.Cu") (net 6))
 (segment (start 128.27 85.09) (end 144.145 85.09) (width 0.2) (layer "F.Cu") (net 5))
 (segment (start 144.78 85.09) (end 145.415 84.455) (width 0.2) (layer "F.Cu") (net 5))
 (segment (start 114.3 71.12) (end 128.27 85.09) (width 0.2) (layer "F.Cu") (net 5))
 (segment (start 144.145 85.09) (end 144.78 85.09) (width 0.2) (layer "F.Cu") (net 5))
 (via (at 145.415 84.455) (size 0.6) (drill 0.3) (layers "F.Cu" "B.Cu") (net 5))
 (segment (start 169.752944 106.68) (end 185.42 106.68) (width 0.2) (layer "B.Cu") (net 5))
 (segment (start 147.527944 84.455) (end 169.752944 106.68) (width 0.2) (layer "B.Cu") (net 5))
 (segment (start 145.415 84.455) (end 147.527944 84.455) (width 0.2) (layer "B.Cu") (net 5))
 (segment (start 114.3 76.2) (end 125.73 87.63) (width 0.2) (layer "B.Cu") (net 13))
 (segment (start 125.73 87.63) (end 146.05 87.63) (width 0.2) (layer "B.Cu") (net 13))
 (segment (start 153.96 95.37) (end 162.295 87.035) (width 0.2) (layer "F.Cu") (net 25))
 (segment (start 114.3 109.22) (end 128.15 95.37) (width 0.2) (layer "F.Cu") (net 25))
 (segment (start 128.15 95.37) (end 153.96 95.37) (width 0.2) (layer "F.Cu") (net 25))
 (segment (start 165.845 83.185) (end 169.695 87.035) (width 0.2) (layer "F.Cu") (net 45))
 (segment (start 136.525 74.93) (end 144.78 83.185) (width 0.2) (layer "F.Cu") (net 45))
 (segment (start 133.35 74.93) (end 136.525 74.93) (width 0.2) (layer "F.Cu") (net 45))
 (segment (start 169.695 87.035) (end 176.795 87.035) (width 0.2) (layer "F.Cu") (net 45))
 (segment (start 144.78 83.185) (end 165.845 83.185) (width 0.2) (layer "F.Cu") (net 45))
 (segment (start 132.08 73.66) (end 133.35 74.93) (width 0.2) (layer "F.Cu") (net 45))
 (segment (start 130.81 97.79) (end 156.54 97.79) (width 0.2) (layer "F.Cu") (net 26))
 (segment (start 114.3 114.3) (end 130.81 97.79) (width 0.2) (layer "F.Cu") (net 26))
 (segment (start 156.54 97.79) (end 162.295 92.035) (width 0.2) (layer "F.Cu") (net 26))
 (segment (start 170.94 81.88) (end 173.99 84.93) (width 0.2) (layer "F.Cu") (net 43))
 (segment (start 132.08 78.74) (end 137.795 78.74) (width 0.2) (layer "F.Cu") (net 43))
 (segment (start 173.99 84.93) (end 173.99 85.09) (width 0.2) (layer "F.Cu") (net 43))
 (segment (start 137.795 78.74) (end 138.43 79.375) (width 0.2) (layer "F.Cu") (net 43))
 (segment (start 144.145 80.01) (end 146.015 81.88) (width 0.2) (layer "F.Cu") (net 43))
 (segment (start 146.015 81.88) (end 170.94 81.88) (width 0.2) (layer "F.Cu") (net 43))
 (segment (start 173.99 85.09) (end 173.99 85.725) (width 0.2) (layer "F.Cu") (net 43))
 (via (at 173.99 85.725) (size 0.6) (drill 0.3) (layers "F.Cu" "B.Cu") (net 43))
 (via (at 144.145 80.01) (size 0.6) (drill 0.3) (layers "F.Cu" "B.Cu") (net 43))
 (via (at 138.43 79.375) (size 0.6) (drill 0.3) (layers "F.Cu" "B.Cu") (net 43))
 (segment (start 173.99 85.725) (end 173.99 89.23) (width 0.2) (layer "B.Cu") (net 43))
 (segment (start 173.99 89.23) (end 176.795 92.035) (width 0.2) (layer "B.Cu") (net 43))
 (segment (start 138.43 79.375) (end 143.51 79.375) (width 0.2) (layer "B.Cu") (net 43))
 (segment (start 143.51 79.375) (end 144.145 80.01) (width 0.2) (layer "B.Cu") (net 43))
 (segment (start 160.995 87.769314) (end 160.995 85.735) (width 0.2) (layer "F.Cu") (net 14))
 (segment (start 167.075 88.97) (end 184.08 88.97) (width 0.2) (layer "F.Cu") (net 14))
 (segment (start 160.995 85.735) (end 163.84 85.735) (width 0.2) (layer "F.Cu") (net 14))
 (segment (start 142.755 90.05) (end 146.924657 94.219657) (width 0.2) (layer "F.Cu") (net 14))
 (segment (start 115.45 87.75) (end 111.35 87.75) (width 0.2) (layer "F.Cu") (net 14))
 (segment (start 118.23 85.21) (end 117.99 85.21) (width 0.2) (layer "F.Cu") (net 14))
 (segment (start 154.544657 94.219657) (end 160.995 87.769314) (width 0.2) (layer "F.Cu") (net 14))
 (segment (start 111.35 87.75) (end 111.35 90.05) (width 0.2) (layer "F.Cu") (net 14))
 (segment (start 184.08 88.97) (end 185.42 87.63) (width 0.2) (layer "F.Cu") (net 14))
 (segment (start 163.84 85.735) (end 167.075 88.97) (width 0.2) (layer "F.Cu") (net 14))
 (segment (start 117.99 85.21) (end 115.45 87.75) (width 0.2) (layer "F.Cu") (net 14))
 (segment (start 111.35 90.05) (end 142.755 90.05) (width 0.2) (layer "F.Cu") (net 14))
 (segment (start 146.924657 94.219657) (end 154.544657 94.219657) (width 0.2) (layer "F.Cu") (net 14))
 (segment (start 114.3 81.28) (end 118.23 85.21) (width 0.2) (layer "F.Cu") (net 14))
 (segment (start 130.175 101.995) (end 131.05 102.87) (width 0.2) (layer "F.Cu") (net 11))
 (segment (start 142.24 102.87) (end 146.05 106.68) (width 0.2) (layer "F.Cu") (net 11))
 (segment (start 118.745 83.185) (end 118.745 86.995) (width 0.2) (layer "F.Cu") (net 11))
 (segment (start 130.175 100.965) (end 130.175 101.995) (width 0.2) (layer "F.Cu") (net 11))
 (segment (start 131.05 102.87) (end 142.24 102.87) (width 0.2) (layer "F.Cu") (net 11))
 (segment (start 114.3 78.74) (end 118.745 83.185) (width 0.2) (layer "F.Cu") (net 11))
 (via (at 130.175 100.965) (size 0.6) (drill 0.3) (layers "F.Cu" "B.Cu") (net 11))
 (via (at 118.745 86.995) (size 0.6) (drill 0.3) (layers "F.Cu" "B.Cu") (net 11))
 (segment (start 120.015 90.805) (end 130.175 100.965) (width 0.2) (layer "B.Cu") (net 11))
 (segment (start 118.745 89.535) (end 120.015 90.805) (width 0.2) (layer "B.Cu") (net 11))
 (segment (start 118.745 86.995) (end 118.745 89.535) (width 0.2) (layer "B.Cu") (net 11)))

